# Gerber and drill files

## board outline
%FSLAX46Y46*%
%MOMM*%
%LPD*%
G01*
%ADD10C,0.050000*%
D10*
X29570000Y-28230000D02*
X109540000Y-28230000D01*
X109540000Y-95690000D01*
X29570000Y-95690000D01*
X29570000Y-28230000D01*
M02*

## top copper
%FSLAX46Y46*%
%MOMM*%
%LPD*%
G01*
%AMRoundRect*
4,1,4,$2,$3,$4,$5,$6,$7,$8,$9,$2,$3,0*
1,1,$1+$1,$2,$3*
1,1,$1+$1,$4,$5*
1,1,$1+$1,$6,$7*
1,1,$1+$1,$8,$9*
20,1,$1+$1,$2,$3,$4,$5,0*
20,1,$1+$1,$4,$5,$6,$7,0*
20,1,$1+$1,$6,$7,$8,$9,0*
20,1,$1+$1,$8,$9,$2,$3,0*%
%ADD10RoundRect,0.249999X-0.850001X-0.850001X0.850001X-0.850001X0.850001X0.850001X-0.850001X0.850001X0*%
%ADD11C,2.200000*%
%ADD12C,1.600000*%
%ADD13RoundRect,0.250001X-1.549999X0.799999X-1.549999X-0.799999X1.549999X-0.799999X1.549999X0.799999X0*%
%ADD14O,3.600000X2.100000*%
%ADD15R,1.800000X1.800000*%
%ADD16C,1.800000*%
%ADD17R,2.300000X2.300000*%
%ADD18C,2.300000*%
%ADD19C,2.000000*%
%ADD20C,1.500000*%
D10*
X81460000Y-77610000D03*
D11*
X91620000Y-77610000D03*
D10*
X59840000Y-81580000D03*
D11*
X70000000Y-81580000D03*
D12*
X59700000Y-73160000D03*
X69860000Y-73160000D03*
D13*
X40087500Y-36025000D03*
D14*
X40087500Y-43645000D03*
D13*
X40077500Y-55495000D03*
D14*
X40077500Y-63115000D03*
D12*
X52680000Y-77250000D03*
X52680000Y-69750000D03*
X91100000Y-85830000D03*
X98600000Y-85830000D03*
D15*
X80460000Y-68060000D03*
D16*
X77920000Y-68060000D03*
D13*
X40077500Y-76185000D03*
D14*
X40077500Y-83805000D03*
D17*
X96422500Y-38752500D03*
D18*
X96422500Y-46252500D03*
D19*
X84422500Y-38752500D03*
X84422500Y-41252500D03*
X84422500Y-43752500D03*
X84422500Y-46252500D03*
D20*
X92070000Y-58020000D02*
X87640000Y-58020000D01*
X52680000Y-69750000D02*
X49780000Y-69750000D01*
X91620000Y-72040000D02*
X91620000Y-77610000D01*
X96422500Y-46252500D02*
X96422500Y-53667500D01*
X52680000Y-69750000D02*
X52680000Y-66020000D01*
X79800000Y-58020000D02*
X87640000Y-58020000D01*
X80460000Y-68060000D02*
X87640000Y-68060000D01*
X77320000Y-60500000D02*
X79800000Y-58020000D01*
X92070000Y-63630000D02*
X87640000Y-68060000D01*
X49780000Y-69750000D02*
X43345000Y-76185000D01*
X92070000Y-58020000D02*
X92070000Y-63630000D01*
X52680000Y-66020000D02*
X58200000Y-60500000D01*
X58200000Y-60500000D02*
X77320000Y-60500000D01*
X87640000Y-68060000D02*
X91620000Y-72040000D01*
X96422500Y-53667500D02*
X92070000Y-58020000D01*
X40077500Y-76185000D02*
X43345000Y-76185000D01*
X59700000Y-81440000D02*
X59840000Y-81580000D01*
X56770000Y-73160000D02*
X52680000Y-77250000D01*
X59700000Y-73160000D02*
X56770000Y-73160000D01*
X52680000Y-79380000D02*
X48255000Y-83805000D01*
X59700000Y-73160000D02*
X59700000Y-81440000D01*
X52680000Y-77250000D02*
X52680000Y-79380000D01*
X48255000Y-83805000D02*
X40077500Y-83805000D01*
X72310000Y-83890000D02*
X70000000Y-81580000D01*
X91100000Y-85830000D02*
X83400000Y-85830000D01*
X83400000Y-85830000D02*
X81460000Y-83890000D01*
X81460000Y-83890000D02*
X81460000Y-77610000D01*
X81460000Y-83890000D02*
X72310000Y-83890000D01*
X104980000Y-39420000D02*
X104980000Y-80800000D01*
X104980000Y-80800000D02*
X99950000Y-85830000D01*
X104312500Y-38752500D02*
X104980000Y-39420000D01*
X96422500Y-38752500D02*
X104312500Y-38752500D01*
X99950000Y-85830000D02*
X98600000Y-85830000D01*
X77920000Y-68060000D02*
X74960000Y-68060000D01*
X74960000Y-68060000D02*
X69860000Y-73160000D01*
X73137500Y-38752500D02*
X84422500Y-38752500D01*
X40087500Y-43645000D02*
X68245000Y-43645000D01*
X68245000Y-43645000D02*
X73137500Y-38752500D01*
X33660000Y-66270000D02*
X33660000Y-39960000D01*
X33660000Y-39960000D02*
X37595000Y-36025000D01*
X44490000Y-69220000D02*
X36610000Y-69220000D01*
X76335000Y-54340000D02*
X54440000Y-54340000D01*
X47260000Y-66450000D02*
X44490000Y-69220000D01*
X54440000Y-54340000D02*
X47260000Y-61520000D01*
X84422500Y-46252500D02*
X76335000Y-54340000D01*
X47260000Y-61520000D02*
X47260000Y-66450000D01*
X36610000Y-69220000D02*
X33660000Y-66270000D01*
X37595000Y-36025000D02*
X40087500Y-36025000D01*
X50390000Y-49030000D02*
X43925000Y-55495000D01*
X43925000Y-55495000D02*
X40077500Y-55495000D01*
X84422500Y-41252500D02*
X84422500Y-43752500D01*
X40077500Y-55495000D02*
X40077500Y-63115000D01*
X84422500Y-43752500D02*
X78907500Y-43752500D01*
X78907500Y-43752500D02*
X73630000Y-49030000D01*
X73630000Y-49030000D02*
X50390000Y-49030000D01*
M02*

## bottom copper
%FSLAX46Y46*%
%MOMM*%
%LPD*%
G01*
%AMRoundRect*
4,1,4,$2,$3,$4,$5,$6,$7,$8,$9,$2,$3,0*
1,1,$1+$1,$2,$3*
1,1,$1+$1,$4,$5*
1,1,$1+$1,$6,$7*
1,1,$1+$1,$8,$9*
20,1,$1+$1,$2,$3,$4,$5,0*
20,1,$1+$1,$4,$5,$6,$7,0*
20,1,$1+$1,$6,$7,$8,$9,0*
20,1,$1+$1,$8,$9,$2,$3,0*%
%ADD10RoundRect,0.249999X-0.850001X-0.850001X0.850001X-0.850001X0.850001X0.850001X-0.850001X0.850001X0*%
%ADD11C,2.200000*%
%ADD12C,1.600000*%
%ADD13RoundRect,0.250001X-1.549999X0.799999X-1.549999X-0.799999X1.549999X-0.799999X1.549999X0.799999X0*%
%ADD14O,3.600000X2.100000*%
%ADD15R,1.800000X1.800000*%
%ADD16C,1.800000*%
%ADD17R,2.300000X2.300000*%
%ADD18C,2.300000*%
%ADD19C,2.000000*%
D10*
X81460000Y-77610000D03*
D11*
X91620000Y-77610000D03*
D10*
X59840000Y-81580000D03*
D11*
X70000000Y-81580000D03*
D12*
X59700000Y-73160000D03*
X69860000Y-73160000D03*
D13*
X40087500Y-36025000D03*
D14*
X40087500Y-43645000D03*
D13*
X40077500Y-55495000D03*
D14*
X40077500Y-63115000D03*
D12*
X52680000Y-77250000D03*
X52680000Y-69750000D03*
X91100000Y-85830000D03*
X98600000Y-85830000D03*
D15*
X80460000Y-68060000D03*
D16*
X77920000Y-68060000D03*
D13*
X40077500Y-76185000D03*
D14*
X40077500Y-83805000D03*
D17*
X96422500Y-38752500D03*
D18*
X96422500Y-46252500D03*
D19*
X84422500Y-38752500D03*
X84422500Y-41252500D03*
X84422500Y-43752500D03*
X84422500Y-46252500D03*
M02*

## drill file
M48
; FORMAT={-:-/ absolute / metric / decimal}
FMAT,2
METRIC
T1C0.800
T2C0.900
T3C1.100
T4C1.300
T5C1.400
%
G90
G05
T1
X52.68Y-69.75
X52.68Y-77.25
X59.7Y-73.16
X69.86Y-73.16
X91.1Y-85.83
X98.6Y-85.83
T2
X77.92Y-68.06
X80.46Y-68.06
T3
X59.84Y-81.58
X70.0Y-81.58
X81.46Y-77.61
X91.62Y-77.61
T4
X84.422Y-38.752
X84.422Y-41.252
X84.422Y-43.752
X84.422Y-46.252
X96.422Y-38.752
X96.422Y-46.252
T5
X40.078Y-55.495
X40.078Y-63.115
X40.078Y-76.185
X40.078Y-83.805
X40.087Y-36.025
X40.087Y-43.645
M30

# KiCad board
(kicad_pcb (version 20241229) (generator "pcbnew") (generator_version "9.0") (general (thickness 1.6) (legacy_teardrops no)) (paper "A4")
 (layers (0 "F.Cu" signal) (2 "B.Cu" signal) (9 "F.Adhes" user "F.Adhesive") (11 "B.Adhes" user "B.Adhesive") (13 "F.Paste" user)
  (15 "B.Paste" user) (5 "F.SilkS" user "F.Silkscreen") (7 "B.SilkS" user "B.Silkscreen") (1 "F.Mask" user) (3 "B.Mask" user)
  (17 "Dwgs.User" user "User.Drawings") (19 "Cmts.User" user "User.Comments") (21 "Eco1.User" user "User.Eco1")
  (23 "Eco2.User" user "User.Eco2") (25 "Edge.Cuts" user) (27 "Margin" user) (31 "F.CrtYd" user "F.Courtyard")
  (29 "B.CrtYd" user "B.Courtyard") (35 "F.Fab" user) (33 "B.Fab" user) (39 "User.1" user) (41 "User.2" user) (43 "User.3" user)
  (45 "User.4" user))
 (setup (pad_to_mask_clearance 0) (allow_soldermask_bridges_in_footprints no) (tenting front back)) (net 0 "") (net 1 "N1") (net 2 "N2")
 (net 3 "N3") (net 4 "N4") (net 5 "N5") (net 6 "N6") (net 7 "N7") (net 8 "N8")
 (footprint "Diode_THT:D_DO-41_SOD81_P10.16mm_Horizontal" (layer "F.Cu") (at 81.46 77.61)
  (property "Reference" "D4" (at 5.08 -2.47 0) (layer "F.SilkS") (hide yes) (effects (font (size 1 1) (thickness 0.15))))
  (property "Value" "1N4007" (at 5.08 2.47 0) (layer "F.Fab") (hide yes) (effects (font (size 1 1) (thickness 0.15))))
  (pad "1" thru_hole roundrect (at 0 0) (size 2.2 2.2) (drill 1.1) (layers "*.Cu" "*.Mask") (remove_unused_layers no)
   (roundrect_rratio 0.113636) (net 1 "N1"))
  (pad "2" thru_hole circle (at 10.16 0) (size 2.2 2.2) (drill 1.1) (layers "*.Cu" "*.Mask") (remove_unused_layers no) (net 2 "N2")))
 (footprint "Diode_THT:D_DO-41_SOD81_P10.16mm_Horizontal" (layer "F.Cu") (at 59.84 81.58)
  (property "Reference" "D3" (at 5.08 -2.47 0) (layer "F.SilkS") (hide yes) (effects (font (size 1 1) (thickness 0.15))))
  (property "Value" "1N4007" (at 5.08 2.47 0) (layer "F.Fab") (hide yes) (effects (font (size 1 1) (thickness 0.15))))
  (pad "1" thru_hole roundrect (at 0 0) (size 2.2 2.2) (drill 1.1) (layers "*.Cu" "*.Mask") (remove_unused_layers no)
   (roundrect_rratio 0.113636) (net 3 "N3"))
  (pad "2" thru_hole circle (at 10.16 0) (size 2.2 2.2) (drill 1.1) (layers "*.Cu" "*.Mask") (remove_unused_layers no) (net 1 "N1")))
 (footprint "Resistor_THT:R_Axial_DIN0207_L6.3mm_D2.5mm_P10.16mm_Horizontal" (layer "F.Cu") (at 59.7 73.16)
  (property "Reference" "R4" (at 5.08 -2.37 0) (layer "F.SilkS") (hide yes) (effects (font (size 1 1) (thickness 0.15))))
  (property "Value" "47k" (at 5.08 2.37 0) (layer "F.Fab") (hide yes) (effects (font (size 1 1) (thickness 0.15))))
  (pad "1" thru_hole circle (at 0 0) (size 1.6 1.6) (drill 0.8) (layers "*.Cu" "*.Mask") (remove_unused_layers no) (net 3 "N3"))
  (pad "2" thru_hole circle (at 10.16 0) (size 1.6 1.6) (drill 0.8) (layers "*.Cu" "*.Mask") (remove_unused_layers no) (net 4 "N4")))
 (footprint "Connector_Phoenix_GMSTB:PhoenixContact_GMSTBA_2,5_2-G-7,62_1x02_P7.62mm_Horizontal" (layer "F.Cu") (at 40.0875 36.025 -90)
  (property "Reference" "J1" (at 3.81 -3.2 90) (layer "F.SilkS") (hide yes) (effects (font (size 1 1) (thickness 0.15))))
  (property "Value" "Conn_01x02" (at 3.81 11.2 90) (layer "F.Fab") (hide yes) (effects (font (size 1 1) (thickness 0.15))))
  (pad "1" thru_hole roundrect (at 0 0 270) (size 2.1 3.6) (drill 1.4) (layers "*.Cu" "*.Mask") (remove_unused_layers no)
   (roundrect_rratio 0.119048) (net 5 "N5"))
  (pad "2" thru_hole oval (at 7.62 0 270) (size 2.1 3.6) (drill 1.4) (layers "*.Cu" "*.Mask") (remove_unused_layers no) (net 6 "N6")))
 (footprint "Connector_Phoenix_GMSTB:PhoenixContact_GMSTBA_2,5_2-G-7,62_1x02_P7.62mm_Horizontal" (layer "F.Cu") (at 40.0775 55.495 -90)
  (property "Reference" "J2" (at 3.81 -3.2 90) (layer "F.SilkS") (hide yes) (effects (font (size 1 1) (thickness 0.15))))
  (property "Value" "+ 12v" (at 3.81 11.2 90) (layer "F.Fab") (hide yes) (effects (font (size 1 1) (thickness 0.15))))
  (pad "1" thru_hole roundrect (at 0 0 270) (size 2.1 3.6) (drill 1.4) (layers "*.Cu" "*.Mask") (remove_unused_layers no)
   (roundrect_rratio 0.119048) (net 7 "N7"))
  (pad "2" thru_hole oval (at 7.62 0 270) (size 2.1 3.6) (drill 1.4) (layers "*.Cu" "*.Mask") (remove_unused_layers no) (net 7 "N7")))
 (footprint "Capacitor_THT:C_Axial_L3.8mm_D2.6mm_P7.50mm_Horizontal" (layer "F.Cu") (at 52.68 77.25 90)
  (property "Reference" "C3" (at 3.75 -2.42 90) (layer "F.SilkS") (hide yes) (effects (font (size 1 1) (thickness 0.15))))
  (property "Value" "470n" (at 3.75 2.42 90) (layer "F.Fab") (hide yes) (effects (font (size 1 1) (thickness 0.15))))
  (pad "1" thru_hole circle (at 0 0 90) (size 1.6 1.6) (drill 0.8) (layers "*.Cu" "*.Mask") (remove_unused_layers no) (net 3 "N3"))
  (pad "2" thru_hole circle (at 7.5 0 90) (size 1.6 1.6) (drill 0.8) (layers "*.Cu" "*.Mask") (remove_unused_layers no) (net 2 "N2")))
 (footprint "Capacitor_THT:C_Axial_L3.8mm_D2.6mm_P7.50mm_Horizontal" (layer "F.Cu") (at 91.1 85.83)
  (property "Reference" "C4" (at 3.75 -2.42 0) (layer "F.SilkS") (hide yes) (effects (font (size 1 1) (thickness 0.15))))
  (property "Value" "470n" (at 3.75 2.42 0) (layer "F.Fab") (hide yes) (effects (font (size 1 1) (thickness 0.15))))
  (pad "1" thru_hole circle (at 0 0) (size 1.6 1.6) (drill 0.8) (layers "*.Cu" "*.Mask") (remove_unused_layers no) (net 1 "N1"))
  (pad "2" thru_hole circle (at 7.5 0) (size 1.6 1.6) (drill 0.8) (layers "*.Cu" "*.Mask") (remove_unused_layers no) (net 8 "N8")))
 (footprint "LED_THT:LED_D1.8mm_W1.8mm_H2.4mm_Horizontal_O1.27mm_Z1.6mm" (layer "F.Cu") (at 80.46 68.06 180)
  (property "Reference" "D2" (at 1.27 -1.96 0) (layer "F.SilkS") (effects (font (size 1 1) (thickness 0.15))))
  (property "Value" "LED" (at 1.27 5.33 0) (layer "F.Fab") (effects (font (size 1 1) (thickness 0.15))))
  (pad "1" thru_hole rect (at 0 0 180) (size 1.8 1.8) (drill 0.9) (layers "*.Cu" "*.Mask") (remove_unused_layers no) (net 2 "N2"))
  (pad "2" thru_hole circle (at 2.54 0 180) (size 1.8 1.8) (drill 0.9) (layers "*.Cu" "*.Mask") (remove_unused_layers no) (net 4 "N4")))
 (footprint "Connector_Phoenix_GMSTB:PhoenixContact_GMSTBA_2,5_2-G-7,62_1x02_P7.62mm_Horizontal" (layer "F.Cu") (at 40.0775 76.185 -90)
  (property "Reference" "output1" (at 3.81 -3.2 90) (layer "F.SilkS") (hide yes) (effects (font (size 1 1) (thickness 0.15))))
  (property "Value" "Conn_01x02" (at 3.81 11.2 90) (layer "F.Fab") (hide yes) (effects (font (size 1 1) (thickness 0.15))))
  (pad "1" thru_hole roundrect (at 0 0 270) (size 2.1 3.6) (drill 1.4) (layers "*.Cu" "*.Mask") (remove_unused_layers no)
   (roundrect_rratio 0.119048) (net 2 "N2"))
  (pad "2" thru_hole oval (at 7.62 0 270) (size 2.1 3.6) (drill 1.4) (layers "*.Cu" "*.Mask") (remove_unused_layers no) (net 3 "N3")))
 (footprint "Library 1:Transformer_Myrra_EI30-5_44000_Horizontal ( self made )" (layer "F.Cu") (at 79.4225 32.7525 -90)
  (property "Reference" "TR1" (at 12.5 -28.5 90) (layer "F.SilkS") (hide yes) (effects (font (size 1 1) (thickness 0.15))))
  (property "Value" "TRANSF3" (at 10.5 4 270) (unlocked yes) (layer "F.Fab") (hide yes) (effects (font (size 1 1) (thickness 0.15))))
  (pad "1" thru_hole rect (at 6 -17 270) (size 2.3 2.3) (drill 1.3) (layers "*.Cu" "*.Mask") (remove_unused_layers no) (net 8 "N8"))
  (pad "2" thru_hole circle (at 13.5 -17 270) (size 2.3 2.3) (drill 1.3) (layers "*.Cu" "*.Mask") (remove_unused_layers no) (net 2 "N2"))
  (pad "3" thru_hole circle (at 6 -5 270) (size 2 2) (drill 1.3) (layers "*.Cu" "*.Mask") (remove_unused_layers no) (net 6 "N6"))
  (pad "4" thru_hole circle (at 8.5 -5 270) (size 2 2) (drill 1.3) (layers "*.Cu" "*.Mask") (remove_unused_layers no) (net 7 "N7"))
  (pad "5" thru_hole circle (at 11 -5 270) (size 2 2) (drill 1.3) (layers "*.Cu" "*.Mask") (remove_unused_layers no) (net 7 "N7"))
  (pad "6" thru_hole circle (at 13.5 -5 270) (size 2 2) (drill 1.3) (layers "*.Cu" "*.Mask") (remove_unused_layers no) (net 5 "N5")))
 (gr_rect (start 29.57 28.23) (end 109.54 95.69) (stroke (width 0.05) (type default)) (fill no) (layer "Edge.Cuts"))
 (segment (start 92.07 58.02) (end 87.64 58.02) (width 1.5) (layer "F.Cu") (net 2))
 (segment (start 52.68 69.75) (end 49.78 69.75) (width 1.5) (layer "F.Cu") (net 2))
 (segment (start 91.62 72.04) (end 91.62 77.61) (width 1.5) (layer "F.Cu") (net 2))
 (segment (start 96.4225 46.2525) (end 96.4225 53.6675) (width 1.5) (layer "F.Cu") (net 2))
 (segment (start 52.68 69.75) (end 52.68 66.02) (width 1.5) (layer "F.Cu") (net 2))
 (segment (start 79.8 58.02) (end 87.64 58.02) (width 1.5) (layer "F.Cu") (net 2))
 (segment (start 80.46 68.06) (end 87.64 68.06) (width 1.5) (layer "F.Cu") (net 2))
 (segment (start 77.32 60.5) (end 79.8 58.02) (width 1.5) (layer "F.Cu") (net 2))
 (segment (start 92.07 63.63) (end 87.64 68.06) (width 1.5) (layer "F.Cu") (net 2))
 (segment (start 49.78 69.75) (end 43.345 76.185) (width 1.5) (layer "F.Cu") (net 2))
 (segment (start 92.07 58.02) (end 92.07 63.63) (width 1.5) (layer "F.Cu") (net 2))
 (segment (start 52.68 66.02) (end 58.2 60.5) (width 1.5) (layer "F.Cu") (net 2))
 (segment (start 58.2 60.5) (end 77.32 60.5) (width 1.5) (layer "F.Cu") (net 2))
 (segment (start 87.64 68.06) (end 91.62 72.04) (width 1.5) (layer "F.Cu") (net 2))
 (segment (start 96.4225 53.6675) (end 92.07 58.02) (width 1.5) (layer "F.Cu") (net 2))
 (segment (start 40.0775 76.185) (end 43.345 76.185) (width 1.5) (layer "F.Cu") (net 2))
 (segment (start 59.7 81.44) (end 59.84 81.58) (width 1.5) (layer "F.Cu") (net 3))
 (segment (start 56.77 73.16) (end 52.68 77.25) (width 1.5) (layer "F.Cu") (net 3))
 (segment (start 59.7 73.16) (end 56.77 73.16) (width 1.5) (layer "F.Cu") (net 3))
 (segment (start 52.68 79.38) (end 48.255 83.805) (width 1.5) (layer "F.Cu") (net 3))
 (segment (start 59.7 73.16) (end 59.7 81.44) (width 1.5) (layer "F.Cu") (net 3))
 (segment (start 52.68 77.25) (end 52.68 79.38) (width 1.5) (layer "F.Cu") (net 3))
 (segment (start 48.255 83.805) (end 40.0775 83.805) (width 1.5) (layer "F.Cu") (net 3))
 (segment (start 72.31 83.89) (end 70 81.58) (width 1.5) (layer "F.Cu") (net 1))
 (segment (start 91.1 85.83) (end 83.4 85.83) (width 1.5) (layer "F.Cu") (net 1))
 (segment (start 83.4 85.83) (end 81.46 83.89) (width 1.5) (layer "F.Cu") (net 1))
 (segment (start 81.46 83.89) (end 81.46 77.61) (width 1.5) (layer "F.Cu") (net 1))
 (segment (start 81.46 83.89) (end 72.31 83.89) (width 1.5) (layer "F.Cu") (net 1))
 (segment (start 104.98 39.42) (end 104.98 80.8) (width 1.5) (layer "F.Cu") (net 8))
 (segment (start 104.98 80.8) (end 99.95 85.83) (width 1.5) (layer "F.Cu") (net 8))
 (segment (start 104.3125 38.7525) (end 104.98 39.42) (width 1.5) (layer "F.Cu") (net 8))
 (segment (start 96.4225 38.7525) (end 104.3125 38.7525) (width 1.5) (layer "F.Cu") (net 8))
 (segment (start 99.95 85.83) (end 98.6 85.83) (width 1.5) (layer "F.Cu") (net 8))
 (segment (start 77.92 68.06) (end 74.96 68.06) (width 1.5) (layer "F.Cu") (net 4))
 (segment (start 74.96 68.06) (end 69.86 73.16) (width 1.5) (layer "F.Cu") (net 4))
 (segment (start 73.1375 38.7525) (end 84.4225 38.7525) (width 1.5) (layer "F.Cu") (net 6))
 (segment (start 40.0875 43.645) (end 68.245 43.645) (width 1.5) (layer "F.Cu") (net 6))
 (segment (start 68.245 43.645) (end 73.1375 38.7525) (width 1.5) (layer "F.Cu") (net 6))
 (segment (start 33.66 66.27) (end 33.66 39.96) (width 1.5) (layer "F.Cu") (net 5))
 (segment (start 33.66 39.96) (end 37.595 36.025) (width 1.5) (layer "F.Cu") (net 5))
 (segment (start 44.49 69.22) (end 36.61 69.22) (width 1.5) (layer "F.Cu") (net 5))
 (segment (start 76.335 54.34) (end 54.44 54.34) (width 1.5) (layer "F.Cu") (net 5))
 (segment (start 47.26 66.45) (end 44.49 69.22) (width 1.5) (layer "F.Cu") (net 5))
 (segment (start 54.44 54.34) (end 47.26 61.52) (width 1.5) (layer "F.Cu") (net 5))
 (segment (start 84.4225 46.2525) (end 76.335 54.34) (width 1.5) (layer "F.Cu") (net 5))
 (segment (start 47.26 61.52) (end 47.26 66.45) (width 1.5) (layer "F.Cu") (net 5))
 (segment (start 36.61 69.22) (end 33.66 66.27) (width 1.5) (layer "F.Cu") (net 5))
 (segment (start 37.595 36.025) (end 40.0875 36.025) (width 1.5) (layer "F.Cu") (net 5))
 (segment (start 50.39 49.03) (end 43.925 55.495) (width 1.5) (layer "F.Cu") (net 7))
 (segment (start 43.925 55.495) (end 40.0775 55.495) (width 1.5) (layer "F.Cu") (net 7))
 (segment (start 84.4225 41.2525) (end 84.4225 43.7525) (width 1.5) (layer "F.Cu") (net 7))
 (segment (start 40.0775 55.495) (end 40.0775 63.115) (width 1.5) (layer "F.Cu") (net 7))
 (segment (start 84.4225 43.7525) (end 78.9075 43.7525) (width 1.5) (layer "F.Cu") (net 7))
 (segment (start 78.9075 43.7525) (end 73.63 49.03) (width 1.5) (layer "F.Cu") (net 7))
 (segment (start 73.63 49.03) (end 50.39 49.03) (width 1.5) (layer "F.Cu") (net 7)))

